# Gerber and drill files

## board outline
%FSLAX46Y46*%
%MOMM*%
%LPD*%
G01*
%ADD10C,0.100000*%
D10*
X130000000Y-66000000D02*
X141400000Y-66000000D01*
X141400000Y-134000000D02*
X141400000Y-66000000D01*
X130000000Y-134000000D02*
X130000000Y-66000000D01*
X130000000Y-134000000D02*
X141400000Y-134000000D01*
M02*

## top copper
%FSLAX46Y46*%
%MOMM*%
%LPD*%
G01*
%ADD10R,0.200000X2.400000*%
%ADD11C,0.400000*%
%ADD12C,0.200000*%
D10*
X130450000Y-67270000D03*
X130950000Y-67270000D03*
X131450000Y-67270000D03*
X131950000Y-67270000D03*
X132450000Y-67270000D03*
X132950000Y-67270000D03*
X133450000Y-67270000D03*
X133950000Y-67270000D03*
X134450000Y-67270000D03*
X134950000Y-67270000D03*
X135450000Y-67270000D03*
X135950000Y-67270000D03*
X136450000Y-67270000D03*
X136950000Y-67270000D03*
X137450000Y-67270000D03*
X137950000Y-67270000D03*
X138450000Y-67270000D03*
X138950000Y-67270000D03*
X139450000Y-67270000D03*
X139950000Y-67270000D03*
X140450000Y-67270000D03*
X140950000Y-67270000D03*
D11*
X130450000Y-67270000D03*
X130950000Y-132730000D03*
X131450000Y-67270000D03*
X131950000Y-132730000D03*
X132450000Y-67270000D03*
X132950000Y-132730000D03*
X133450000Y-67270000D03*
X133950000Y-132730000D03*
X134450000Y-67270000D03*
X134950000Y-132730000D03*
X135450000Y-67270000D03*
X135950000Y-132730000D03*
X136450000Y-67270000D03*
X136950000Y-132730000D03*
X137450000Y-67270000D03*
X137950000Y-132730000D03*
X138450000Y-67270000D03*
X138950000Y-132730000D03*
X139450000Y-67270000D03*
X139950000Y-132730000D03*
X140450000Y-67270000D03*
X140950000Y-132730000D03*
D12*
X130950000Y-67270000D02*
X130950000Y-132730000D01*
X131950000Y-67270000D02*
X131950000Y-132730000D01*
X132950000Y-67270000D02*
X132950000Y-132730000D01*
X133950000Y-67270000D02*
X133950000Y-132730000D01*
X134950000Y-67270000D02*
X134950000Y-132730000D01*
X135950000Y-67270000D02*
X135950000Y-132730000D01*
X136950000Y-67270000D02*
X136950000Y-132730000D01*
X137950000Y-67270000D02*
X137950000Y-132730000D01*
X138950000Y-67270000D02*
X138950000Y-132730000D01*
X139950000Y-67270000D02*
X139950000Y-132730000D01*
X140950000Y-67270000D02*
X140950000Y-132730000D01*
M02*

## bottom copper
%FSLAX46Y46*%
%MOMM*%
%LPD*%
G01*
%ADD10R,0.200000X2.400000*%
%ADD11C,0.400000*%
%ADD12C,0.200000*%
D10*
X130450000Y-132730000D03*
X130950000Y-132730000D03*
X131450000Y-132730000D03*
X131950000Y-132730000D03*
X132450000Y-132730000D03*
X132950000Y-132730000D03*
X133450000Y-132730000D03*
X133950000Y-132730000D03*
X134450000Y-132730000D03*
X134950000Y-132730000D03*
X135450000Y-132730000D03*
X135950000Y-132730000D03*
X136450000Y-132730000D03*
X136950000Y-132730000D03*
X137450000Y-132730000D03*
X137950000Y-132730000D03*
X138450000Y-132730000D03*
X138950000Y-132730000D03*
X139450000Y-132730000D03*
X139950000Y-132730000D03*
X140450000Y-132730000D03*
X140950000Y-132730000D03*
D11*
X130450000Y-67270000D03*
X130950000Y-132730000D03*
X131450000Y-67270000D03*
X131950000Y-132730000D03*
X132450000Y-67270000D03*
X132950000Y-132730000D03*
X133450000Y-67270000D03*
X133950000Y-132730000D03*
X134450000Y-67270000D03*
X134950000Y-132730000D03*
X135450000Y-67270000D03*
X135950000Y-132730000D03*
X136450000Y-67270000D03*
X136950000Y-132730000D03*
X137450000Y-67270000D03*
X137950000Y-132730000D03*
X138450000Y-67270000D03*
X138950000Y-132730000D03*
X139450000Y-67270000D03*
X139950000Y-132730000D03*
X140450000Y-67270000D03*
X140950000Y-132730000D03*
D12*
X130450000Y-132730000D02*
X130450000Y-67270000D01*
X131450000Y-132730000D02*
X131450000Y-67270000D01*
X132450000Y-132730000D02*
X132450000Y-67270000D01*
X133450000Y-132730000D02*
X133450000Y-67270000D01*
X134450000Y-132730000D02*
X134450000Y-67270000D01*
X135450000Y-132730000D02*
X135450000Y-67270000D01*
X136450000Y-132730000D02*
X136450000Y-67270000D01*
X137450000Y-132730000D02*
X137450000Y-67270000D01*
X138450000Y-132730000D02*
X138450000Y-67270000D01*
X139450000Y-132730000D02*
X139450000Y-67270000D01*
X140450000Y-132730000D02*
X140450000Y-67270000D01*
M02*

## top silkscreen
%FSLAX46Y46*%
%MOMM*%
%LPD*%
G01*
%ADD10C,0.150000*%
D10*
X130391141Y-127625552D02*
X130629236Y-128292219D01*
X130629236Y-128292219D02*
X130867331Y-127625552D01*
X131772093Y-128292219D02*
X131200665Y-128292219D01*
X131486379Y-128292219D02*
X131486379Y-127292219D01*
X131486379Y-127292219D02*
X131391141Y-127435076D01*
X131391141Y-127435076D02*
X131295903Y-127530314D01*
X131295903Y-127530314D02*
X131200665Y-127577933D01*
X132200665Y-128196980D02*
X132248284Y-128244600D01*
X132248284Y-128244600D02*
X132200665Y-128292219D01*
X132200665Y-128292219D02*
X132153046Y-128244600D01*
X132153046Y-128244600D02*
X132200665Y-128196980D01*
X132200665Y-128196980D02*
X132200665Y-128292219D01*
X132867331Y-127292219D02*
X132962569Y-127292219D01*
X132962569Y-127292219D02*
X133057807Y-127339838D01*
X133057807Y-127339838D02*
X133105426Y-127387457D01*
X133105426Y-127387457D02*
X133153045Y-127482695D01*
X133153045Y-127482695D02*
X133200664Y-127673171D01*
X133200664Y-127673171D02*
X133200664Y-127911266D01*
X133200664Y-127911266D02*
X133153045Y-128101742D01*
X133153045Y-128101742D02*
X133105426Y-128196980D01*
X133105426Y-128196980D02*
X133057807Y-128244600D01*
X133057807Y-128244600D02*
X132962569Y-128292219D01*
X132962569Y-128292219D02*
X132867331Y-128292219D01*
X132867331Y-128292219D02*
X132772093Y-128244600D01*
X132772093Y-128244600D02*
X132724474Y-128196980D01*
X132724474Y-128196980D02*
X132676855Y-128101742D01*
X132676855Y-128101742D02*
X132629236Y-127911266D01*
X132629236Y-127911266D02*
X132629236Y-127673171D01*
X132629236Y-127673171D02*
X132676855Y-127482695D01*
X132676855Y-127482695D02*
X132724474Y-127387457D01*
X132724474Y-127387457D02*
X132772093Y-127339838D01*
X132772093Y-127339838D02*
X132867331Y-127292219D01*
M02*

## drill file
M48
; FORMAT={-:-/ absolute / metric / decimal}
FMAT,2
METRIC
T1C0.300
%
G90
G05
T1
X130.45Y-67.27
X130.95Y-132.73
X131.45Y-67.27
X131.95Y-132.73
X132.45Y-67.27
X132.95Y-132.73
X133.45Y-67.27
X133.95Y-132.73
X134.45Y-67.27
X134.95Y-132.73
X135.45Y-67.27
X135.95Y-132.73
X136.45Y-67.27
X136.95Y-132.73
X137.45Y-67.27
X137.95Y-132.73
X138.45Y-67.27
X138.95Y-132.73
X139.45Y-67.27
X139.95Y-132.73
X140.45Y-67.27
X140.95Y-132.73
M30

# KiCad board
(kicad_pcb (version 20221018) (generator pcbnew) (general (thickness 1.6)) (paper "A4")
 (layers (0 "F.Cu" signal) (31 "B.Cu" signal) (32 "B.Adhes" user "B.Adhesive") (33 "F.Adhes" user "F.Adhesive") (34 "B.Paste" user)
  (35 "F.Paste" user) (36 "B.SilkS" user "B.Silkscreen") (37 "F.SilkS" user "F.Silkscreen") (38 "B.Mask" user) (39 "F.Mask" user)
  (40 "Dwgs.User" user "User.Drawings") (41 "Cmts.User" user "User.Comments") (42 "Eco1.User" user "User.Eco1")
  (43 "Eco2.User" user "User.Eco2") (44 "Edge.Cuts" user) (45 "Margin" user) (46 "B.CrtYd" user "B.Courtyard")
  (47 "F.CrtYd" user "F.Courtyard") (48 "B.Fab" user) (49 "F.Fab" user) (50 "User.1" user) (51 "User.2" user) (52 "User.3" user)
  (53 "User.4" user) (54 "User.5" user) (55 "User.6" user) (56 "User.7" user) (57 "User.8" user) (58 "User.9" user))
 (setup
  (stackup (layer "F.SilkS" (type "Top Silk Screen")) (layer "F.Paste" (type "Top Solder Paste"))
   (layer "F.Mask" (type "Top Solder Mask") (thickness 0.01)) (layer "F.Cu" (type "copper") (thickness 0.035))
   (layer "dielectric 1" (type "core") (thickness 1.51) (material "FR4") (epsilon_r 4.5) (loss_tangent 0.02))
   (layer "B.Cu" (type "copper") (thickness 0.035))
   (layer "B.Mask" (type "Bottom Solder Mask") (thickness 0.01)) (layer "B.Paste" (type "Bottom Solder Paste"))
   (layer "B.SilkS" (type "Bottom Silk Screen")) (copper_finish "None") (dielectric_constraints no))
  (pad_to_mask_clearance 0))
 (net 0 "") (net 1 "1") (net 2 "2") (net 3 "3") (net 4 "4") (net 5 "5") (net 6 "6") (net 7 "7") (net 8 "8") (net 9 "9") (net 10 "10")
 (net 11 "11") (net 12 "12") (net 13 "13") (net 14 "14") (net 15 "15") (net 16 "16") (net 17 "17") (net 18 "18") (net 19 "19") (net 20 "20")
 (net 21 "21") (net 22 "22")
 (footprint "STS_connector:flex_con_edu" (layer "F.Cu") (at 130 70.62)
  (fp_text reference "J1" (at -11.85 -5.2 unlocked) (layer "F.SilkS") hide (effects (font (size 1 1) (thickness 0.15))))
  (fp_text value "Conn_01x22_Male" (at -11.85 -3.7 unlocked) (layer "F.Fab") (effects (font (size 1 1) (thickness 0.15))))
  (pad "1" smd rect (at 0.45 -3.35) (size 0.2 2.4) (layers "F.Cu" "F.Paste" "F.Mask") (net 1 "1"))
  (pad "2" smd rect (at 0.95 -3.35) (size 0.2 2.4) (layers "F.Cu" "F.Paste" "F.Mask") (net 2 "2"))
  (pad "3" smd rect (at 1.45 -3.35) (size 0.2 2.4) (layers "F.Cu" "F.Paste" "F.Mask") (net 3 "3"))
  (pad "4" smd rect (at 1.95 -3.35) (size 0.2 2.4) (layers "F.Cu" "F.Paste" "F.Mask") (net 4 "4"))
  (pad "5" smd rect (at 2.45 -3.35) (size 0.2 2.4) (layers "F.Cu" "F.Paste" "F.Mask") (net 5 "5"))
  (pad "6" smd rect (at 2.95 -3.35) (size 0.2 2.4) (layers "F.Cu" "F.Paste" "F.Mask") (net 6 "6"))
  (pad "7" smd rect (at 3.45 -3.35) (size 0.2 2.4) (layers "F.Cu" "F.Paste" "F.Mask") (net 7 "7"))
  (pad "8" smd rect (at 3.95 -3.35) (size 0.2 2.4) (layers "F.Cu" "F.Paste" "F.Mask") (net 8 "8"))
  (pad "9" smd rect (at 4.45 -3.35) (size 0.2 2.4) (layers "F.Cu" "F.Paste" "F.Mask") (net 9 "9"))
  (pad "10" smd rect (at 4.95 -3.35) (size 0.2 2.4) (layers "F.Cu" "F.Paste" "F.Mask") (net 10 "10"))
  (pad "11" smd rect (at 5.45 -3.35) (size 0.2 2.4) (layers "F.Cu" "F.Paste" "F.Mask") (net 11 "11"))
  (pad "12" smd rect (at 5.95 -3.35) (size 0.2 2.4) (layers "F.Cu" "F.Paste" "F.Mask") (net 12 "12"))
  (pad "13" smd rect (at 6.45 -3.35) (size 0.2 2.4) (layers "F.Cu" "F.Paste" "F.Mask") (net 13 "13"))
  (pad "14" smd rect (at 6.95 -3.35) (size 0.2 2.4) (layers "F.Cu" "F.Paste" "F.Mask") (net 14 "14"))
  (pad "15" smd rect (at 7.45 -3.35) (size 0.2 2.4) (layers "F.Cu" "F.Paste" "F.Mask") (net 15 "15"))
  (pad "16" smd rect (at 7.95 -3.35) (size 0.2 2.4) (layers "F.Cu" "F.Paste" "F.Mask") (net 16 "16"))
  (pad "17" smd rect (at 8.45 -3.35) (size 0.2 2.4) (layers "F.Cu" "F.Paste" "F.Mask") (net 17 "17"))
  (pad "18" smd rect (at 8.95 -3.35) (size 0.2 2.4) (layers "F.Cu" "F.Paste" "F.Mask") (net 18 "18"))
  (pad "19" smd rect (at 9.45 -3.35) (size 0.2 2.4) (layers "F.Cu" "F.Paste" "F.Mask") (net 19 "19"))
  (pad "20" smd rect (at 9.95 -3.35) (size 0.2 2.4) (layers "F.Cu" "F.Paste" "F.Mask") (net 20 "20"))
  (pad "21" smd rect (at 10.45 -3.35) (size 0.2 2.4) (layers "F.Cu" "F.Paste" "F.Mask") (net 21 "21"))
  (pad "22" smd rect (at 10.95 -3.35) (size 0.2 2.4) (layers "F.Cu" "F.Paste" "F.Mask") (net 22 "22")))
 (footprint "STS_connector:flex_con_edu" (layer "B.Cu") (at 130 129.38)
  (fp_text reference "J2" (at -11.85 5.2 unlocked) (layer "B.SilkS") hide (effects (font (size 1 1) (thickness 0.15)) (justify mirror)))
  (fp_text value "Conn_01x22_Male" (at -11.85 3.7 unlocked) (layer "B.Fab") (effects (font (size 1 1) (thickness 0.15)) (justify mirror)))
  (pad "1" smd rect (at 0.45 3.35) (size 0.2 2.4) (layers "B.Cu" "B.Paste" "B.Mask") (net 1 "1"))
  (pad "2" smd rect (at 0.95 3.35) (size 0.2 2.4) (layers "B.Cu" "B.Paste" "B.Mask") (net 2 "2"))
  (pad "3" smd rect (at 1.45 3.35) (size 0.2 2.4) (layers "B.Cu" "B.Paste" "B.Mask") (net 3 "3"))
  (pad "4" smd rect (at 1.95 3.35) (size 0.2 2.4) (layers "B.Cu" "B.Paste" "B.Mask") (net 4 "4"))
  (pad "5" smd rect (at 2.45 3.35) (size 0.2 2.4) (layers "B.Cu" "B.Paste" "B.Mask") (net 5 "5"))
  (pad "6" smd rect (at 2.95 3.35) (size 0.2 2.4) (layers "B.Cu" "B.Paste" "B.Mask") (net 6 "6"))
  (pad "7" smd rect (at 3.45 3.35) (size 0.2 2.4) (layers "B.Cu" "B.Paste" "B.Mask") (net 7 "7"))
  (pad "8" smd rect (at 3.95 3.35) (size 0.2 2.4) (layers "B.Cu" "B.Paste" "B.Mask") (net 8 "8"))
  (pad "9" smd rect (at 4.45 3.35) (size 0.2 2.4) (layers "B.Cu" "B.Paste" "B.Mask") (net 9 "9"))
  (pad "10" smd rect (at 4.95 3.35) (size 0.2 2.4) (layers "B.Cu" "B.Paste" "B.Mask") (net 10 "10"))
  (pad "11" smd rect (at 5.45 3.35) (size 0.2 2.4) (layers "B.Cu" "B.Paste" "B.Mask") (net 11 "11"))
  (pad "12" smd rect (at 5.95 3.35) (size 0.2 2.4) (layers "B.Cu" "B.Paste" "B.Mask") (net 12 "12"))
  (pad "13" smd rect (at 6.45 3.35) (size 0.2 2.4) (layers "B.Cu" "B.Paste" "B.Mask") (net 13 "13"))
  (pad "14" smd rect (at 6.95 3.35) (size 0.2 2.4) (layers "B.Cu" "B.Paste" "B.Mask") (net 14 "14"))
  (pad "15" smd rect (at 7.45 3.35) (size 0.2 2.4) (layers "B.Cu" "B.Paste" "B.Mask") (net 15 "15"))
  (pad "16" smd rect (at 7.95 3.35) (size 0.2 2.4) (layers "B.Cu" "B.Paste" "B.Mask") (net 16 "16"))
  (pad "17" smd rect (at 8.45 3.35) (size 0.2 2.4) (layers "B.Cu" "B.Paste" "B.Mask") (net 17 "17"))
  (pad "18" smd rect (at 8.95 3.35) (size 0.2 2.4) (layers "B.Cu" "B.Paste" "B.Mask") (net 18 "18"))
  (pad "19" smd rect (at 9.45 3.35) (size 0.2 2.4) (layers "B.Cu" "B.Paste" "B.Mask") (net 19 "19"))
  (pad "20" smd rect (at 9.95 3.35) (size 0.2 2.4) (layers "B.Cu" "B.Paste" "B.Mask") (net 20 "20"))
  (pad "21" smd rect (at 10.45 3.35) (size 0.2 2.4) (layers "B.Cu" "B.Paste" "B.Mask") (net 21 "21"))
  (pad "22" smd rect (at 10.95 3.35) (size 0.2 2.4) (layers "B.Cu" "B.Paste" "B.Mask") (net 22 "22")))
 (gr_line (start 130 66) (end 141.4 66) (stroke (width 0.1) (type solid)) (layer "Edge.Cuts"))
 (gr_line (start 141.4 134) (end 141.4 66) (stroke (width 0.1) (type solid)) (layer "Edge.Cuts"))
 (gr_line (start 130 134) (end 130 66) (stroke (width 0.1) (type solid)) (layer "Edge.Cuts"))
 (gr_line (start 130 134) (end 141.4 134) (stroke (width 0.1) (type solid)) (layer "Edge.Cuts"))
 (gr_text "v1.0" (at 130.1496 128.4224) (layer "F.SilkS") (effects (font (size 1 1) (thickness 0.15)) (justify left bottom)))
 (via (at 130.45 67.27) (size 0.4) (drill 0.3) (layers "F.Cu" "B.Cu") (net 1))
 (segment (start 130.45 132.73) (end 130.45 67.27) (width 0.2) (layer "B.Cu") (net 1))
 (segment (start 130.95 67.27) (end 130.95 132.73) (width 0.2) (layer "F.Cu") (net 2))
 (via (at 130.95 132.73) (size 0.4) (drill 0.3) (layers "F.Cu" "B.Cu") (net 2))
 (via (at 131.45 67.27) (size 0.4) (drill 0.3) (layers "F.Cu" "B.Cu") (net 3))
 (segment (start 131.45 132.73) (end 131.45 67.27) (width 0.2) (layer "B.Cu") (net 3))
 (segment (start 131.95 67.27) (end 131.95 132.73) (width 0.2) (layer "F.Cu") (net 4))
 (via (at 131.95 132.73) (size 0.4) (drill 0.3) (layers "F.Cu" "B.Cu") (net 4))
 (via (at 132.45 67.27) (size 0.4) (drill 0.3) (layers "F.Cu" "B.Cu") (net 5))
 (segment (start 132.45 132.73) (end 132.45 67.27) (width 0.2) (layer "B.Cu") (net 5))
 (segment (start 132.95 67.27) (end 132.95 132.73) (width 0.2) (layer "F.Cu") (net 6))
 (via (at 132.95 132.73) (size 0.4) (drill 0.3) (layers "F.Cu" "B.Cu") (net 6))
 (via (at 133.45 67.27) (size 0.4) (drill 0.3) (layers "F.Cu" "B.Cu") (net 7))
 (segment (start 133.45 132.73) (end 133.45 67.27) (width 0.2) (layer "B.Cu") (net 7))
 (segment (start 133.95 67.27) (end 133.95 132.73) (width 0.2) (layer "F.Cu") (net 8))
 (via (at 133.95 132.73) (size 0.4) (drill 0.3) (layers "F.Cu" "B.Cu") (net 8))
 (via (at 134.45 67.27) (size 0.4) (drill 0.3) (layers "F.Cu" "B.Cu") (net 9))
 (segment (start 134.45 132.73) (end 134.45 67.27) (width 0.2) (layer "B.Cu") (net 9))
 (segment (start 134.95 67.27) (end 134.95 132.73) (width 0.2) (layer "F.Cu") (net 10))
 (via (at 134.95 132.73) (size 0.4) (drill 0.3) (layers "F.Cu" "B.Cu") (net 10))
 (via (at 135.45 67.27) (size 0.4) (drill 0.3) (layers "F.Cu" "B.Cu") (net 11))
 (segment (start 135.45 132.73) (end 135.45 67.27) (width 0.2) (layer "B.Cu") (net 11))
 (segment (start 135.95 67.27) (end 135.95 132.73) (width 0.2) (layer "F.Cu") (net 12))
 (via (at 135.95 132.73) (size 0.4) (drill 0.3) (layers "F.Cu" "B.Cu") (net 12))
 (via (at 136.45 67.27) (size 0.4) (drill 0.3) (layers "F.Cu" "B.Cu") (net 13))
 (segment (start 136.45 132.73) (end 136.45 67.27) (width 0.2) (layer "B.Cu") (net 13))
 (segment (start 136.95 67.27) (end 136.95 132.73) (width 0.2) (layer "F.Cu") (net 14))
 (via (at 136.95 132.73) (size 0.4) (drill 0.3) (layers "F.Cu" "B.Cu") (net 14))
 (via (at 137.45 67.27) (size 0.4) (drill 0.3) (layers "F.Cu" "B.Cu") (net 15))
 (segment (start 137.45 132.73) (end 137.45 67.27) (width 0.2) (layer "B.Cu") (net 15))
 (segment (start 137.95 67.27) (end 137.95 132.73) (width 0.2) (layer "F.Cu") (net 16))
 (via (at 137.95 132.73) (size 0.4) (drill 0.3) (layers "F.Cu" "B.Cu") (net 16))
 (via (at 138.45 67.27) (size 0.4) (drill 0.3) (layers "F.Cu" "B.Cu") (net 17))
 (segment (start 138.45 132.73) (end 138.45 67.27) (width 0.2) (layer "B.Cu") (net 17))
 (segment (start 138.95 67.27) (end 138.95 132.73) (width 0.2) (layer "F.Cu") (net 18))
 (via (at 138.95 132.73) (size 0.4) (drill 0.3) (layers "F.Cu" "B.Cu") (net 18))
 (via (at 139.45 67.27) (size 0.4) (drill 0.3) (layers "F.Cu" "B.Cu") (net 19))
 (segment (start 139.45 132.73) (end 139.45 67.27) (width 0.2) (layer "B.Cu") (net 19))
 (segment (start 139.95 67.27) (end 139.95 132.73) (width 0.2) (layer "F.Cu") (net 20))
 (via (at 139.95 132.73) (size 0.4) (drill 0.3) (layers "F.Cu" "B.Cu") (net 20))
 (via (at 140.45 67.27) (size 0.4) (drill 0.3) (layers "F.Cu" "B.Cu") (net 21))
 (segment (start 140.45 132.73) (end 140.45 67.27) (width 0.2) (layer "B.Cu") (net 21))
 (segment (start 140.95 67.27) (end 140.95 132.73) (width 0.2) (layer "F.Cu") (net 22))
 (via (at 140.95 132.73) (size 0.4) (drill 0.3) (layers "F.Cu" "B.Cu") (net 22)))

